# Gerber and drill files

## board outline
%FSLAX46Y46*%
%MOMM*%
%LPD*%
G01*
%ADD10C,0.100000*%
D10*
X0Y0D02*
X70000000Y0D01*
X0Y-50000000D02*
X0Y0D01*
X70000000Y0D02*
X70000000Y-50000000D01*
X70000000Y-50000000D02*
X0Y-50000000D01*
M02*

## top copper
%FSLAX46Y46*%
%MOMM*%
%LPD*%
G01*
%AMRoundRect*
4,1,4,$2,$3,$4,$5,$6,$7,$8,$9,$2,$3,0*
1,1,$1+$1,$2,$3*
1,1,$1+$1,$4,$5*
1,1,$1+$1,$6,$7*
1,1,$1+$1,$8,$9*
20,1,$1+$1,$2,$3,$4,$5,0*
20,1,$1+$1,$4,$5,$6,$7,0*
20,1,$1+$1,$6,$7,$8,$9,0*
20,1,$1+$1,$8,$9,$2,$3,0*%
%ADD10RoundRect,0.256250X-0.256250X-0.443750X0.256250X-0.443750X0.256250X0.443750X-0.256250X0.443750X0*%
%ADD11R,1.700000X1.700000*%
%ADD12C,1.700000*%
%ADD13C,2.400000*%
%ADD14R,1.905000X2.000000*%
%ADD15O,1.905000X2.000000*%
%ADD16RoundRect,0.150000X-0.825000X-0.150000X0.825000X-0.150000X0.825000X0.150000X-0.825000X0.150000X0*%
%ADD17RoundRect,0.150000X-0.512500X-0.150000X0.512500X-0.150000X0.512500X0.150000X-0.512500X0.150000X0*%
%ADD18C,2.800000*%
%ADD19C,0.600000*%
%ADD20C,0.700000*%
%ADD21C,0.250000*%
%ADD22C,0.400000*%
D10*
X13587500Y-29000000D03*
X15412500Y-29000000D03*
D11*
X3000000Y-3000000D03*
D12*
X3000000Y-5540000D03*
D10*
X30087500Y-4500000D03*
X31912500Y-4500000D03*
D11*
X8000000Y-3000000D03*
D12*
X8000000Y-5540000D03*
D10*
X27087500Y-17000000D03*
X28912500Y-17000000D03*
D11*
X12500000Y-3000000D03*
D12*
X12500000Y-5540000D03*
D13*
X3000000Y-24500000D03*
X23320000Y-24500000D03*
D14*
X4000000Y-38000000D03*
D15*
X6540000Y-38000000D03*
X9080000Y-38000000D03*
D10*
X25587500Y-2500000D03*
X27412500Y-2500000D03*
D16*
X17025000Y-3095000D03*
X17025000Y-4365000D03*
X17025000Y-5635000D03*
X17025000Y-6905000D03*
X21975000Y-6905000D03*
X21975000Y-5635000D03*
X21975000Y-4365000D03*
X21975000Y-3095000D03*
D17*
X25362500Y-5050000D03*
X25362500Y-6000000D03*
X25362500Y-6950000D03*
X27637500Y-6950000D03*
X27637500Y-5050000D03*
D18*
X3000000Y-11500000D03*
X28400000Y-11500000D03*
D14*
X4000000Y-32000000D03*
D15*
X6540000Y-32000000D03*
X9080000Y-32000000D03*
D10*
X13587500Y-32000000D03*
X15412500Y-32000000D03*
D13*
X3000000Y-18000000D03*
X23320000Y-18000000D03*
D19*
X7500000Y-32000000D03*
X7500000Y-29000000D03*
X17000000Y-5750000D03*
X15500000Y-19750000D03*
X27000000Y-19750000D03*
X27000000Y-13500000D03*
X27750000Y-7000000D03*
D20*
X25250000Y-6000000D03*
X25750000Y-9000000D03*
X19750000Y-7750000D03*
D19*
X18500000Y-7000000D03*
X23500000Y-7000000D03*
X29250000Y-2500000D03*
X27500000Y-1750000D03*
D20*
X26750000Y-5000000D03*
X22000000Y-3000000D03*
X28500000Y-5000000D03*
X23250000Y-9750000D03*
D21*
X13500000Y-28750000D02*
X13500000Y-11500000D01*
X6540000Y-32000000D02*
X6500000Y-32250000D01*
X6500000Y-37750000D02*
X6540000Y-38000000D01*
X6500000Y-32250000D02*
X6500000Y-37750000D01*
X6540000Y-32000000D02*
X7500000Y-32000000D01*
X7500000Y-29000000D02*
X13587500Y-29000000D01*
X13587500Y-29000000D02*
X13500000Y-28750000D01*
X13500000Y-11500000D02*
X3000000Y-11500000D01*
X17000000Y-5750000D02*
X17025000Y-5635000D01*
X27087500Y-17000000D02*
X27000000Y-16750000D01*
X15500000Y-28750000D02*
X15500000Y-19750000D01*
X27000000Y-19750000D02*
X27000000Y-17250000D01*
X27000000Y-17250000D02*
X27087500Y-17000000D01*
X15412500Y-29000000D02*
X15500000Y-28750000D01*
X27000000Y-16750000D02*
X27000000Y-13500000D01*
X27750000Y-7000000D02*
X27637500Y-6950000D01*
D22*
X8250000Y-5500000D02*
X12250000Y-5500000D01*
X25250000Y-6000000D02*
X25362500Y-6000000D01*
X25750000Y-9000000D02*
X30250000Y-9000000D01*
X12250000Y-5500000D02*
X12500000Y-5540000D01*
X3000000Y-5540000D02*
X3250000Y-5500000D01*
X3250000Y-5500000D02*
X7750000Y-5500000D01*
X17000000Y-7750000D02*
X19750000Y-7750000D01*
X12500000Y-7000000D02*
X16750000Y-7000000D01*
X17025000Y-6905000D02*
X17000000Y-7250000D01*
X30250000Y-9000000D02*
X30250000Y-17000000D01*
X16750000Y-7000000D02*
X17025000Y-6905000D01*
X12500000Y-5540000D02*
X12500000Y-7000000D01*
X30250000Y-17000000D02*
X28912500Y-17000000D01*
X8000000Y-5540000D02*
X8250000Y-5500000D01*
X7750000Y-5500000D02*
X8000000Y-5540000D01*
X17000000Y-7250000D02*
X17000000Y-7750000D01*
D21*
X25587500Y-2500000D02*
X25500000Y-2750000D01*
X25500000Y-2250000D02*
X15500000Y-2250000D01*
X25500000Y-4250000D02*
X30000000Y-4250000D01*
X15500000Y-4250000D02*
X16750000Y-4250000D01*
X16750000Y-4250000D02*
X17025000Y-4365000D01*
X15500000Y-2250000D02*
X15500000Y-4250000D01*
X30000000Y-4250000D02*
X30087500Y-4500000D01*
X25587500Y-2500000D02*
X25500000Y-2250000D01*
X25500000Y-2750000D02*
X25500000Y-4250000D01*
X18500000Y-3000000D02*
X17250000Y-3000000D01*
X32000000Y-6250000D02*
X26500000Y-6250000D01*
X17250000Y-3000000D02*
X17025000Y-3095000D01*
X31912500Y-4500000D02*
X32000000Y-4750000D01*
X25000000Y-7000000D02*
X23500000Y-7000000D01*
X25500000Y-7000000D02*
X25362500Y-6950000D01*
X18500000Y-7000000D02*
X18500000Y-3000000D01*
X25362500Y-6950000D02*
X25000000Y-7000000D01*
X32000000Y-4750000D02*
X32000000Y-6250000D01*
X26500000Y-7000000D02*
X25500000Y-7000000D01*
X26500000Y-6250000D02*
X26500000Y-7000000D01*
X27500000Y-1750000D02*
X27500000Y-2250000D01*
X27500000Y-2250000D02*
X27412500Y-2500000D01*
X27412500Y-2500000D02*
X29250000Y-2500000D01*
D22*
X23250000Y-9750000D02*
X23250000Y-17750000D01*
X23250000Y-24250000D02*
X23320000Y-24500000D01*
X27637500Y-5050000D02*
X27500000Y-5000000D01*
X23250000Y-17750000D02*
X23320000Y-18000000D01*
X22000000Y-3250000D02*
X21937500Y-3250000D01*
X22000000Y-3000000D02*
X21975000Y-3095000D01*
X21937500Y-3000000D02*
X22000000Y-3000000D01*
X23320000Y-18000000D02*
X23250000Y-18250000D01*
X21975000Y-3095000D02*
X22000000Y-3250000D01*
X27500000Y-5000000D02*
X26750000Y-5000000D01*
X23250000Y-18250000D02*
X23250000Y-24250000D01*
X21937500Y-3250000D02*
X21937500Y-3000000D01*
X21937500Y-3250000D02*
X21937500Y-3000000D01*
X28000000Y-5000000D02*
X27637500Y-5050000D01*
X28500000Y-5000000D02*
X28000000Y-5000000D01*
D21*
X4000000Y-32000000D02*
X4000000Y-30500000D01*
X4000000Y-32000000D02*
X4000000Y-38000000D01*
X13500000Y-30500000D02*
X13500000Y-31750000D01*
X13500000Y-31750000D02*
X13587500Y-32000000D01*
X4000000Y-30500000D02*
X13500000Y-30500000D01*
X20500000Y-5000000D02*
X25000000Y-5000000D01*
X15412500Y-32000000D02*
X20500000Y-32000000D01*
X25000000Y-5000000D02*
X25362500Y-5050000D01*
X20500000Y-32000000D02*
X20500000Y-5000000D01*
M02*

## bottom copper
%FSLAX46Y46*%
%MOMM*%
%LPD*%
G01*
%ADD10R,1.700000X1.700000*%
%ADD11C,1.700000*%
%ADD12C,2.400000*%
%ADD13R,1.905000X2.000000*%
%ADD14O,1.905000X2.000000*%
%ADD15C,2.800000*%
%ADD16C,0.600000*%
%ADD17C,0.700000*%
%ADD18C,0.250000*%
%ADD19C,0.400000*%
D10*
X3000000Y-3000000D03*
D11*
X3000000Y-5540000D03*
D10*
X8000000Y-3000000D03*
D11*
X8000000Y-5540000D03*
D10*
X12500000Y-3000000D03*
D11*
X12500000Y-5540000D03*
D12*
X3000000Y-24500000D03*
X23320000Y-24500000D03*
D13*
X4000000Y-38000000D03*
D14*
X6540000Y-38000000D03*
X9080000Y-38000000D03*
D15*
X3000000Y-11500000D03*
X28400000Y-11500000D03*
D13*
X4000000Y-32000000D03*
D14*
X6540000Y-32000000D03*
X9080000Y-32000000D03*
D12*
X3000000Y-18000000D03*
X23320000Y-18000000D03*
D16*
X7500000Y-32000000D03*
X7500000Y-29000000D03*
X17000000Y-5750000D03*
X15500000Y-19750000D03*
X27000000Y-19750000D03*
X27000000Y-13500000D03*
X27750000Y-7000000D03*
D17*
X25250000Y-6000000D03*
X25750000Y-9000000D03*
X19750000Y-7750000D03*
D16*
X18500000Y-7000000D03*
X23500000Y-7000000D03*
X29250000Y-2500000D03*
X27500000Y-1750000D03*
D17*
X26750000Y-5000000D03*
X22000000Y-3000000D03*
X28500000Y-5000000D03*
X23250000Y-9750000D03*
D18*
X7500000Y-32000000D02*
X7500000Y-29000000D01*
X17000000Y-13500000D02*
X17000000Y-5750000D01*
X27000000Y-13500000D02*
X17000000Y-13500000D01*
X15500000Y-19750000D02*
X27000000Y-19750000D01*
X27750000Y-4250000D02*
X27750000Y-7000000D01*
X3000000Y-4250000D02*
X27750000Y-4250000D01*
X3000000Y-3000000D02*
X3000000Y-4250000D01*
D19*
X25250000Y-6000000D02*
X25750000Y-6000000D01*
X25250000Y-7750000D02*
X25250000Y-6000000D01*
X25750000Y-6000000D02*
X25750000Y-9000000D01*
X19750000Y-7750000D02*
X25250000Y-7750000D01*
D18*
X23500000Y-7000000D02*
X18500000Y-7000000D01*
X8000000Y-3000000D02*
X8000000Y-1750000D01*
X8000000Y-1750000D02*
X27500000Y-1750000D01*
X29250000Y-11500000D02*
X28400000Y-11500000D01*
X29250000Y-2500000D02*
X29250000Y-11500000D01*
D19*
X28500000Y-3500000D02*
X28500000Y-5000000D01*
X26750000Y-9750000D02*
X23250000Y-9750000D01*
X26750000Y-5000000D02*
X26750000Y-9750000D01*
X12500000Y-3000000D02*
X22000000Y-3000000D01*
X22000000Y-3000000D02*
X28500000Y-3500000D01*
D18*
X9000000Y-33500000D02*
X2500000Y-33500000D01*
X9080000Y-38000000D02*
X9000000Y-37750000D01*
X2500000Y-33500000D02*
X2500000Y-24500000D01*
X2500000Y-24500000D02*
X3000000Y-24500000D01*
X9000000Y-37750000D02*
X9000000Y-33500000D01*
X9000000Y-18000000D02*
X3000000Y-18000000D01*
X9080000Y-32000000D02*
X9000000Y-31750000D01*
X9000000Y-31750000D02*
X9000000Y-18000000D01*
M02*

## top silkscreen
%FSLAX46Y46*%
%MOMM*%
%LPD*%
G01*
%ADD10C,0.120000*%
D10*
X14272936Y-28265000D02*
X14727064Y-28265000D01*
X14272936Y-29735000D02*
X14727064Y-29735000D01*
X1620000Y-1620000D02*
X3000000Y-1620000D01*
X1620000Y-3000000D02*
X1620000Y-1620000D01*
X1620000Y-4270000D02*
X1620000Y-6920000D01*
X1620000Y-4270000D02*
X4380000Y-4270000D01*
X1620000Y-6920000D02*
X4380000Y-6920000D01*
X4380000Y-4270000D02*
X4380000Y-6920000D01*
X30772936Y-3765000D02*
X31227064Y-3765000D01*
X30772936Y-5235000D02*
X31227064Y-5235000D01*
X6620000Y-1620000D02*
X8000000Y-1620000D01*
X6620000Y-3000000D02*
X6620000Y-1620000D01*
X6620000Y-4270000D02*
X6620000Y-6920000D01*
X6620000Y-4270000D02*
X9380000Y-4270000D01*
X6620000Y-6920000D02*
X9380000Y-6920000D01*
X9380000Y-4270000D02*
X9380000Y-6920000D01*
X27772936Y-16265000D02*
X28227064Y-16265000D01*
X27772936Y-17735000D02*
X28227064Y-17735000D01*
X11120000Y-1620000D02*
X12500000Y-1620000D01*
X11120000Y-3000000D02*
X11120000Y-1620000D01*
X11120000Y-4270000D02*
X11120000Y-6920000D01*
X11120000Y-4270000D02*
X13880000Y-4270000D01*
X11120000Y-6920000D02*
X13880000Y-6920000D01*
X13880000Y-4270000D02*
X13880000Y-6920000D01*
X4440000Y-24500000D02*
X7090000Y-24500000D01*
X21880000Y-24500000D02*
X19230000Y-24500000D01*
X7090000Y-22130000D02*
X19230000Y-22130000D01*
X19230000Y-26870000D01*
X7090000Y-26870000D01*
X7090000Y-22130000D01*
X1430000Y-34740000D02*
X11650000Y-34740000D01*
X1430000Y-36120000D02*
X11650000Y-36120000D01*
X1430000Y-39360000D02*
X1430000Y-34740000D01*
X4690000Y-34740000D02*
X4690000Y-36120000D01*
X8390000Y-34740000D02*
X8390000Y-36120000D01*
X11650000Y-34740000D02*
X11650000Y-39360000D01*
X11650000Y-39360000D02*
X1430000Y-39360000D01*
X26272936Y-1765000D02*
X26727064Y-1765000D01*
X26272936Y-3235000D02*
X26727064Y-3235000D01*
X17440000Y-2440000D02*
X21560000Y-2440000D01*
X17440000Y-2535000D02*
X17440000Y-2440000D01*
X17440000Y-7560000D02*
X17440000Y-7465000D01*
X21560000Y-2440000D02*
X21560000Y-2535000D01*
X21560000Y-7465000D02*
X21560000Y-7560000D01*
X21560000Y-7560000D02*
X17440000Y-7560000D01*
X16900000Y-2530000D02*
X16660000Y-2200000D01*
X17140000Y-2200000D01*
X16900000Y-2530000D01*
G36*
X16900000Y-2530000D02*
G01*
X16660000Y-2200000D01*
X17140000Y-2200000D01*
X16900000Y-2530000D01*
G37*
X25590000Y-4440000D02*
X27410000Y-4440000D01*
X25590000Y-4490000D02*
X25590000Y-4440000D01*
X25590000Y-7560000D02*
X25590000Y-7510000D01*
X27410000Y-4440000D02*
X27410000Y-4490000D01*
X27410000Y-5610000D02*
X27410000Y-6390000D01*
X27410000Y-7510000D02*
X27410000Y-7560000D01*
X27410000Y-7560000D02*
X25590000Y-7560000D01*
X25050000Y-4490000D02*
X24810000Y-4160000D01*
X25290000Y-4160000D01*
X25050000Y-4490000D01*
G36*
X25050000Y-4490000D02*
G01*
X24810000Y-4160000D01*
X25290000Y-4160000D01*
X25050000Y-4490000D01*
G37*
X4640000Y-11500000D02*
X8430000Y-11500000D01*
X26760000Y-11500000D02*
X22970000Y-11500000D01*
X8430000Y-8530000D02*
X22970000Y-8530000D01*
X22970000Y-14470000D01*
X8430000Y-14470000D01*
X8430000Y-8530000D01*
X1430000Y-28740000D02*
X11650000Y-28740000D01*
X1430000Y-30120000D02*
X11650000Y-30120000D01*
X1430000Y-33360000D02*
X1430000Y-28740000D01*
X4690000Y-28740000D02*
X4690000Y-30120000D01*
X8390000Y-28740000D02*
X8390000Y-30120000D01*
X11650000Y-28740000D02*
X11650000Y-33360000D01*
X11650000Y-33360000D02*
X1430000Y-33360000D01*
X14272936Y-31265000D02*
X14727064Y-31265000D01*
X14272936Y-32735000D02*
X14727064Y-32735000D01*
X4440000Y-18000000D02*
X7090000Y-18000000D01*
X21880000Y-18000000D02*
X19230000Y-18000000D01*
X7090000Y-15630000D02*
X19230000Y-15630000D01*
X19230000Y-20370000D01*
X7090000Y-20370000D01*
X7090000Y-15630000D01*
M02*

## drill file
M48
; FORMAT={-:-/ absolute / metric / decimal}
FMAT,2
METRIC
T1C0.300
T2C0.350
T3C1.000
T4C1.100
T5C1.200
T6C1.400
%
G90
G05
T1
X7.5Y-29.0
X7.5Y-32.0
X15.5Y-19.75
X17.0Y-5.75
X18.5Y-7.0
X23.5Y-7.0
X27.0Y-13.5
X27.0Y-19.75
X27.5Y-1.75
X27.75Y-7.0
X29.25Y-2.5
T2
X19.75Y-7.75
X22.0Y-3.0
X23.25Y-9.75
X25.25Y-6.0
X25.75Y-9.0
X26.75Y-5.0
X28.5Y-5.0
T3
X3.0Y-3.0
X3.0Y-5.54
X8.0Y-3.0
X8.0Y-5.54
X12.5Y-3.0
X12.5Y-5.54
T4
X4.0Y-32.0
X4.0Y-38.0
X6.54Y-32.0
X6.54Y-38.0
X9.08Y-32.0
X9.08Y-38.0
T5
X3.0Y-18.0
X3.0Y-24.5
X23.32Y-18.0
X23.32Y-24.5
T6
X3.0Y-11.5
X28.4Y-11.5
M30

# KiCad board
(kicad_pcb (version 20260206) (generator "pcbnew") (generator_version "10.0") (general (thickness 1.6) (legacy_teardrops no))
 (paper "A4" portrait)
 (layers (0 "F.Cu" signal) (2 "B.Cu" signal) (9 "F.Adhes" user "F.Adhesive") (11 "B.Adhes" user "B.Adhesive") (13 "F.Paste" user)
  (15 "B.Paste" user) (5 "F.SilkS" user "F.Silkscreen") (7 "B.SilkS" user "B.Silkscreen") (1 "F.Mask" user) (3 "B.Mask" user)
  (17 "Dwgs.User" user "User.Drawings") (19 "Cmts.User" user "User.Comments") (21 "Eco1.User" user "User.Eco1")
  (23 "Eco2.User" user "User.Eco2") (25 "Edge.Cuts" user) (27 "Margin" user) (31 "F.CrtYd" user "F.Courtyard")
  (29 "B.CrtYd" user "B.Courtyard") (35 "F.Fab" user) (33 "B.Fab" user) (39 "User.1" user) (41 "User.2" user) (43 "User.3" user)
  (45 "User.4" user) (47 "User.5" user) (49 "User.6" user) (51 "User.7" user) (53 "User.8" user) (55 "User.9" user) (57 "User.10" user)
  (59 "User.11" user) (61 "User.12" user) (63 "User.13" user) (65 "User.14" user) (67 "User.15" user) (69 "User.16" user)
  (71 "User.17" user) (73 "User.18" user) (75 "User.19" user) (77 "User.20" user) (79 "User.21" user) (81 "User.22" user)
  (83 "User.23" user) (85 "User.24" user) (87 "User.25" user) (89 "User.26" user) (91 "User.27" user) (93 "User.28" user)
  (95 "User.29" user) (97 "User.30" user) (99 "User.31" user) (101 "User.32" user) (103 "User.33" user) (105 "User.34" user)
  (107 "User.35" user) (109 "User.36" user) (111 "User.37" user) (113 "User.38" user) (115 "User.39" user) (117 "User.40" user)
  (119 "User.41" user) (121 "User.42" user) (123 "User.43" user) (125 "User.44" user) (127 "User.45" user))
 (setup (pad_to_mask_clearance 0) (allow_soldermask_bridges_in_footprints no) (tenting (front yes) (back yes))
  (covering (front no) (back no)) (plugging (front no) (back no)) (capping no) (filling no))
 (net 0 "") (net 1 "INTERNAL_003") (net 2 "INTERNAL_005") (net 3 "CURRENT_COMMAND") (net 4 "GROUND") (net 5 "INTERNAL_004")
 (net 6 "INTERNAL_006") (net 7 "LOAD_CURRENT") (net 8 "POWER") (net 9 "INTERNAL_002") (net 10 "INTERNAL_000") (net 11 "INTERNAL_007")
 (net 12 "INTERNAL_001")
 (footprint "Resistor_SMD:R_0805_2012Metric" (layer "F.Cu") (at 14.5 29)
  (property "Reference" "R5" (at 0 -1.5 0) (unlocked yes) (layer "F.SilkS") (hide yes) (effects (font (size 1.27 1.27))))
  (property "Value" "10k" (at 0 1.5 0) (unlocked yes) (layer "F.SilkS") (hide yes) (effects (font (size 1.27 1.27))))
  (fp_line (start -0.227064 -0.735) (end 0.227064 -0.735) (stroke (width 0.12) (type solid)) (layer "F.SilkS"))
  (fp_line (start -0.227064 0.735) (end 0.227064 0.735) (stroke (width 0.12) (type solid)) (layer "F.SilkS"))
  (pad "1" smd roundrect (at -0.9125 0) (size 1.025 1.4) (layers "F.Cu" "F.Mask" "F.Paste") (roundrect_rratio 0.25) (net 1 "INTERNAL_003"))
  (pad "2" smd roundrect (at 0.9125 0) (size 1.025 1.4) (layers "F.Cu" "F.Mask" "F.Paste") (roundrect_rratio 0.25) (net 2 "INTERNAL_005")))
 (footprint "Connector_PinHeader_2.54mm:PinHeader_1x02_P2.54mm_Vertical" (layer "F.Cu") (at 3 3)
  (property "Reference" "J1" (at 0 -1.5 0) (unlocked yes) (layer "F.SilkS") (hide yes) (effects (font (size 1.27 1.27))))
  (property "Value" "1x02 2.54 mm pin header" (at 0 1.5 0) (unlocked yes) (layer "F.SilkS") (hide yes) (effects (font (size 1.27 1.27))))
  (fp_line (start -1.38 -1.38) (end 0 -1.38) (stroke (width 0.12) (type solid)) (layer "F.SilkS"))
  (fp_line (start -1.38 0) (end -1.38 -1.38) (stroke (width 0.12) (type solid)) (layer "F.SilkS"))
  (fp_line (start -1.38 1.27) (end -1.38 3.92) (stroke (width 0.12) (type solid)) (layer "F.SilkS"))
  (fp_line (start -1.38 1.27) (end 1.38 1.27) (stroke (width 0.12) (type solid)) (layer "F.SilkS"))
  (fp_line (start -1.38 3.92) (end 1.38 3.92) (stroke (width 0.12) (type solid)) (layer "F.SilkS"))
  (fp_line (start 1.38 1.27) (end 1.38 3.92) (stroke (width 0.12) (type solid)) (layer "F.SilkS"))
  (pad "1" thru_hole rect (at 0 0) (size 1.7 1.7) (drill 1) (layers "*.Cu" "*.Mask") (remove_unused_layers no) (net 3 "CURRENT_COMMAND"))
  (pad "2" thru_hole circle (at 0 2.54) (size 1.7 1.7) (drill 1) (layers "*.Cu" "*.Mask") (remove_unused_layers no) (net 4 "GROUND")))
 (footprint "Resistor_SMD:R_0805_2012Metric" (layer "F.Cu") (at 31 4.5)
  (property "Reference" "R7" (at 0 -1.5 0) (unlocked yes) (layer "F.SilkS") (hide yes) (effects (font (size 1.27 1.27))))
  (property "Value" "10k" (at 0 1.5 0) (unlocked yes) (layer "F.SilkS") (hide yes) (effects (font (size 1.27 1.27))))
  (fp_line (start -0.227064 -0.735) (end 0.227064 -0.735) (stroke (width 0.12) (type solid)) (layer "F.SilkS"))
  (fp_line (start -0.227064 0.735) (end 0.227064 0.735) (stroke (width 0.12) (type solid)) (layer "F.SilkS"))
  (pad "1" smd roundrect (at -0.9125 0) (size 1.025 1.4) (layers "F.Cu" "F.Mask" "F.Paste") (roundrect_rratio 0.25) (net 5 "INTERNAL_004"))
  (pad "2" smd roundrect (at 0.9125 0) (size 1.025 1.4) (layers "F.Cu" "F.Mask" "F.Paste") (roundrect_rratio 0.25) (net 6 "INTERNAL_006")))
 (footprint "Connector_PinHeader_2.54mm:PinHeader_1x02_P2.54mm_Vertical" (layer "F.Cu") (at 8 3)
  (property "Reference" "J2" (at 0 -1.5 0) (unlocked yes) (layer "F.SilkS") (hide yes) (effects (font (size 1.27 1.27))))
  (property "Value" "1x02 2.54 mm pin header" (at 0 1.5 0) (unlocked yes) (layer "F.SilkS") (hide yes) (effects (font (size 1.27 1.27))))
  (fp_line (start -1.38 -1.38) (end 0 -1.38) (stroke (width 0.12) (type solid)) (layer "F.SilkS"))
  (fp_line (start -1.38 0) (end -1.38 -1.38) (stroke (width 0.12) (type solid)) (layer "F.SilkS"))
  (fp_line (start -1.38 1.27) (end -1.38 3.92) (stroke (width 0.12) (type solid)) (layer "F.SilkS"))
  (fp_line (start -1.38 1.27) (end 1.38 1.27) (stroke (width 0.12) (type solid)) (layer "F.SilkS"))
  (fp_line (start -1.38 3.92) (end 1.38 3.92) (stroke (width 0.12) (type solid)) (layer "F.SilkS"))
  (fp_line (start 1.38 1.27) (end 1.38 3.92) (stroke (width 0.12) (type solid)) (layer "F.SilkS"))
  (pad "1" thru_hole rect (at 0 0) (size 1.7 1.7) (drill 1) (layers "*.Cu" "*.Mask") (remove_unused_layers no) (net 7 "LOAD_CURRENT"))
  (pad "2" thru_hole circle (at 0 2.54) (size 1.7 1.7) (drill 1) (layers "*.Cu" "*.Mask") (remove_unused_layers no) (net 4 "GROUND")))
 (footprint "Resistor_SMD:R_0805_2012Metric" (layer "F.Cu") (at 28 17)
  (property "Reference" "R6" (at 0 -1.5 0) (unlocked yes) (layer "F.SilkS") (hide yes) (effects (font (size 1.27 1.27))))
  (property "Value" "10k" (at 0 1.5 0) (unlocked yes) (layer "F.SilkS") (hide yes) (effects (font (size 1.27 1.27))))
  (fp_line (start -0.227064 -0.735) (end 0.227064 -0.735) (stroke (width 0.12) (type solid)) (layer "F.SilkS"))
  (fp_line (start -0.227064 0.735) (end 0.227064 0.735) (stroke (width 0.12) (type solid)) (layer "F.SilkS"))
  (pad "1" smd roundrect (at -0.9125 0) (size 1.025 1.4) (layers "F.Cu" "F.Mask" "F.Paste") (roundrect_rratio 0.25) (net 2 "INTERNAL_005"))
  (pad "2" smd roundrect (at 0.9125 0) (size 1.025 1.4) (layers "F.Cu" "F.Mask" "F.Paste") (roundrect_rratio 0.25) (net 4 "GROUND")))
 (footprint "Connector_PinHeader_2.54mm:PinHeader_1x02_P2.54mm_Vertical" (layer "F.Cu") (at 12.5 3)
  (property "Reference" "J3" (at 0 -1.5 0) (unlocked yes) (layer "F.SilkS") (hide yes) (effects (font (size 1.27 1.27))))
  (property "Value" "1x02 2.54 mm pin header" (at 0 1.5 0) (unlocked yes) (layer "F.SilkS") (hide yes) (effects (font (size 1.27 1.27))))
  (fp_line (start -1.38 -1.38) (end 0 -1.38) (stroke (width 0.12) (type solid)) (layer "F.SilkS"))
  (fp_line (start -1.38 0) (end -1.38 -1.38) (stroke (width 0.12) (type solid)) (layer "F.SilkS"))
  (fp_line (start -1.38 1.27) (end -1.38 3.92) (stroke (width 0.12) (type solid)) (layer "F.SilkS"))
  (fp_line (start -1.38 1.27) (end 1.38 1.27) (stroke (width 0.12) (type solid)) (layer "F.SilkS"))
  (fp_line (start -1.38 3.92) (end 1.38 3.92) (stroke (width 0.12) (type solid)) (layer "F.SilkS"))
  (fp_line (start 1.38 1.27) (end 1.38 3.92) (stroke (width 0.12) (type solid)) (layer "F.SilkS"))
  (pad "1" thru_hole rect (at 0 0) (size 1.7 1.7) (drill 1) (layers "*.Cu" "*.Mask") (remove_unused_layers no) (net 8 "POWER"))
  (pad "2" thru_hole circle (at 0 2.54) (size 1.7 1.7) (drill 1) (layers "*.Cu" "*.Mask") (remove_unused_layers no) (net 4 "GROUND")))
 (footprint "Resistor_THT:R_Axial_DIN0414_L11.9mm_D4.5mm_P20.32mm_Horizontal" (layer "F.Cu") (at 3 24.5)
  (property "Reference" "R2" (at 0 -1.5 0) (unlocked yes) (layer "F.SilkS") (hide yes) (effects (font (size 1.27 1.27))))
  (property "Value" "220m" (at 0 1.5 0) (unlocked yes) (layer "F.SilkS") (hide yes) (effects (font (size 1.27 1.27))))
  (fp_line (start 1.44 0) (end 4.09 0) (stroke (width 0.12) (type solid)) (layer "F.SilkS"))
  (fp_line (start 18.88 0) (end 16.23 0) (stroke (width 0.12) (type solid)) (layer "F.SilkS"))
  (fp_rect (start 4.09 -2.37) (end 16.23 2.37) (stroke (width 0.12) (type solid)) (fill no) (layer "F.SilkS"))
  (pad "1" thru_hole circle (at 0 0) (size 2.4 2.4) (drill 1.2) (layers "*.Cu" "*.Mask") (remove_unused_layers no) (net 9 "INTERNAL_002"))
  (pad "2" thru_hole circle (at 20.32 0) (size 2.4 2.4) (drill 1.2) (layers "*.Cu" "*.Mask") (remove_unused_layers no) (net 8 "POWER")))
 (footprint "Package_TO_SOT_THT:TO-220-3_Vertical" (layer "F.Cu") (at 4 38)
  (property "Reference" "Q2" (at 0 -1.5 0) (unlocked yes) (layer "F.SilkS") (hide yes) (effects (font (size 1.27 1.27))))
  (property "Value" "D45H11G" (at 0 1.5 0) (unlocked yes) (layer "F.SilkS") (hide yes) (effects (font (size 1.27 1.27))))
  (fp_line (start -2.57 -3.26) (end 7.65 -3.26) (stroke (width 0.12) (type solid)) (layer "F.SilkS"))
  (fp_line (start -2.57 -1.88) (end 7.65 -1.88) (stroke (width 0.12) (type solid)) (layer "F.SilkS"))
  (fp_line (start -2.57 1.36) (end -2.57 -3.26) (stroke (width 0.12) (type solid)) (layer "F.SilkS"))
  (fp_line (start 0.69 -3.26) (end 0.69 -1.88) (stroke (width 0.12) (type solid)) (layer "F.SilkS"))
  (fp_line (start 4.39 -3.26) (end 4.39 -1.88) (stroke (width 0.12) (type solid)) (layer "F.SilkS"))
  (fp_line (start 7.65 -3.26) (end 7.65 1.36) (stroke (width 0.12) (type solid)) (layer "F.SilkS"))
  (fp_line (start 7.65 1.36) (end -2.57 1.36) (stroke (width 0.12) (type solid)) (layer "F.SilkS"))
  (pad "1" thru_hole rect (at 0 0) (size 1.905 2) (drill 1.1) (layers "*.Cu" "*.Mask") (remove_unused_layers no) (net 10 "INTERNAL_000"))
  (pad "2" thru_hole oval (at 2.54 0) (size 1.905 2) (drill 1.1) (layers "*.Cu" "*.Mask") (remove_unused_layers no) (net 1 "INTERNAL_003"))
  (pad "3" thru_hole oval (at 5.08 0) (size 1.905 2) (drill 1.1) (layers "*.Cu" "*.Mask") (remove_unused_layers no) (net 9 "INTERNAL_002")))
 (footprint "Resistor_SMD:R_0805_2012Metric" (layer "F.Cu") (at 26.5 2.5)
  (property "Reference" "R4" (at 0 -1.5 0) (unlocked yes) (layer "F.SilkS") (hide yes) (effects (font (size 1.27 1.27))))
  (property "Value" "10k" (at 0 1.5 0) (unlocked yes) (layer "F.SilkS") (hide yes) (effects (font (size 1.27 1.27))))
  (fp_line (start -0.227064 -0.735) (end 0.227064 -0.735) (stroke (width 0.12) (type solid)) (layer "F.SilkS"))
  (fp_line (start -0.227064 0.735) (end 0.227064 0.735) (stroke (width 0.12) (type solid)) (layer "F.SilkS"))
  (pad "1" smd roundrect (at -0.9125 0) (size 1.025 1.4) (layers "F.Cu" "F.Mask" "F.Paste") (roundrect_rratio 0.25) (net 5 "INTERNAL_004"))
  (pad "2" smd roundrect (at 0.9125 0) (size 1.025 1.4) (layers "F.Cu" "F.Mask" "F.Paste") (roundrect_rratio 0.25) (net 7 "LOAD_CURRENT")))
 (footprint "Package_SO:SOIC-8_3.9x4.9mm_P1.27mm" (layer "F.Cu") (at 19.5 5)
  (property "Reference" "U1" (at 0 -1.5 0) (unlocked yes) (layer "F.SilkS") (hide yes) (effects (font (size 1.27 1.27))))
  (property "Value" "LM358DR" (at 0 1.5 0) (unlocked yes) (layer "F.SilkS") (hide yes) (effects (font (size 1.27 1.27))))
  (fp_line (start -2.06 -2.56) (end 2.06 -2.56) (stroke (width 0.12) (type solid)) (layer "F.SilkS"))
  (fp_line (start -2.06 -2.465) (end -2.06 -2.56) (stroke (width 0.12) (type solid)) (layer "F.SilkS"))
  (fp_line (start -2.06 2.56) (end -2.06 2.465) (stroke (width 0.12) (type solid)) (layer "F.SilkS"))
  (fp_line (start 2.06 -2.56) (end 2.06 -2.465) (stroke (width 0.12) (type solid)) (layer "F.SilkS"))
  (fp_line (start 2.06 2.465) (end 2.06 2.56) (stroke (width 0.12) (type solid)) (layer "F.SilkS"))
  (fp_line (start 2.06 2.56) (end -2.06 2.56) (stroke (width 0.12) (type solid)) (layer "F.SilkS"))
  (fp_poly (pts (xy -2.6 -2.47) (xy -2.84 -2.8) (xy -2.36 -2.8)) (stroke (width 0.12) (type solid)) (fill yes) (layer "F.SilkS"))
  (pad "1" smd roundrect (at -2.475 -1.905) (size 1.95 0.6) (layers "F.Cu" "F.Mask" "F.Paste") (roundrect_rratio 0.25)
   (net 6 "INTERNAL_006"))
  (pad "2" smd roundrect (at -2.475 -0.635) (size 1.95 0.6) (layers "F.Cu" "F.Mask" "F.Paste") (roundrect_rratio 0.25)
   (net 5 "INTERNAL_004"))
  (pad "3" smd roundrect (at -2.475 0.635) (size 1.95 0.6) (layers "F.Cu" "F.Mask" "F.Paste") (roundrect_rratio 0.25) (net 2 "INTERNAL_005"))
  (pad "4" smd roundrect (at -2.475 1.905) (size 1.95 0.6) (layers "F.Cu" "F.Mask" "F.Paste") (roundrect_rratio 0.25) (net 4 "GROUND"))
  (pad "5" smd roundrect (at 2.475 1.905) (size 1.95 0.6) (layers "F.Cu" "F.Mask" "F.Paste") (roundrect_rratio 0.25))
  (pad "6" smd roundrect (at 2.475 0.635) (size 1.95 0.6) (layers "F.Cu" "F.Mask" "F.Paste") (roundrect_rratio 0.25))
  (pad "7" smd roundrect (at 2.475 -0.635) (size 1.95 0.6) (layers "F.Cu" "F.Mask" "F.Paste") (roundrect_rratio 0.25))
  (pad "8" smd roundrect (at 2.475 -1.905) (size 1.95 0.6) (layers "F.Cu" "F.Mask" "F.Paste") (roundrect_rratio 0.25) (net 8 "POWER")))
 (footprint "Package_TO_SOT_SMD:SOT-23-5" (layer "F.Cu") (at 26.5 6)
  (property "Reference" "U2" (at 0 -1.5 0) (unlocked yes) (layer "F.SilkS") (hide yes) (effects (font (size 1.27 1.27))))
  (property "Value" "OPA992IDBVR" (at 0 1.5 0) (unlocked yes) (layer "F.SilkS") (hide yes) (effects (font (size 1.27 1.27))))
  (fp_line (start -0.91 -1.56) (end 0.91 -1.56) (stroke (width 0.12) (type solid)) (layer "F.SilkS"))
  (fp_line (start -0.91 -1.51) (end -0.91 -1.56) (stroke (width 0.12) (type solid)) (layer "F.SilkS"))
  (fp_line (start -0.91 1.56) (end -0.91 1.51) (stroke (width 0.12) (type solid)) (layer "F.SilkS"))
  (fp_line (start 0.91 -1.56) (end 0.91 -1.51) (stroke (width 0.12) (type solid)) (layer "F.SilkS"))
  (fp_line (start 0.91 -0.39) (end 0.91 0.39) (stroke (width 0.12) (type solid)) (layer "F.SilkS"))
  (fp_line (start 0.91 1.51) (end 0.91 1.56) (stroke (width 0.12) (type solid)) (layer "F.SilkS"))
  (fp_line (start 0.91 1.56) (end -0.91 1.56) (stroke (width 0.12) (type solid)) (layer "F.SilkS"))
  (fp_poly (pts (xy -1.45 -1.51) (xy -1.69 -1.84) (xy -1.21 -1.84)) (stroke (width 0.12) (type solid)) (fill yes) (layer "F.SilkS"))
  (pad "1" smd roundrect (at -1.1375 -0.95) (size 1.325 0.6) (layers "F.Cu" "F.Mask" "F.Paste") (roundrect_rratio 0.25)
   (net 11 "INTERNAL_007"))
  (pad "2" smd roundrect (at -1.1375 0) (size 1.325 0.6) (layers "F.Cu" "F.Mask" "F.Paste") (roundrect_rratio 0.25) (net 4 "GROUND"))
  (pad "3" smd roundrect (at -1.1375 0.95) (size 1.325 0.6) (layers "F.Cu" "F.Mask" "F.Paste") (roundrect_rratio 0.25)
   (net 6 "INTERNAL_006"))
  (pad "4" smd roundrect (at 1.1375 0.95) (size 1.325 0.6) (layers "F.Cu" "F.Mask" "F.Paste") (roundrect_rratio 0.25)
   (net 3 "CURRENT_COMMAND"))
  (pad "5" smd roundrect (at 1.1375 -0.95) (size 1.325 0.6) (layers "F.Cu" "F.Mask" "F.Paste") (roundrect_rratio 0.25) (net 8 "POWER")))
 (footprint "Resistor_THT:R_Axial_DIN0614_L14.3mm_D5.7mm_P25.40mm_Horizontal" (layer "F.Cu") (at 3 11.5)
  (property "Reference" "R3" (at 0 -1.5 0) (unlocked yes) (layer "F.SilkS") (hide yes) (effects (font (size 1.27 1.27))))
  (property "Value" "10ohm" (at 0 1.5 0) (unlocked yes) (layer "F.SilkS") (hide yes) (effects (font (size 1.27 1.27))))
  (fp_line (start 1.64 0) (end 5.43 0) (stroke (width 0.12) (type solid)) (layer "F.SilkS"))
  (fp_line (start 23.76 0) (end 19.97 0) (stroke (width 0.12) (type solid)) (layer "F.SilkS"))
  (fp_rect (start 5.43 -2.97) (end 19.97 2.97) (stroke (width 0.12) (type solid)) (fill no) (layer "F.SilkS"))
  (pad "1" thru_hole circle (at 0 0) (size 2.8 2.8) (drill 1.4) (layers "*.Cu" "*.Mask") (remove_unused_layers no) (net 1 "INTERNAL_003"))
  (pad "2" thru_hole circle (at 25.4 0) (size 2.8 2.8) (drill 1.4) (layers "*.Cu" "*.Mask") (remove_unused_layers no) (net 7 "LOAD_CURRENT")))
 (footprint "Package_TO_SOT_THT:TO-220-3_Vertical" (layer "F.Cu") (at 4 32)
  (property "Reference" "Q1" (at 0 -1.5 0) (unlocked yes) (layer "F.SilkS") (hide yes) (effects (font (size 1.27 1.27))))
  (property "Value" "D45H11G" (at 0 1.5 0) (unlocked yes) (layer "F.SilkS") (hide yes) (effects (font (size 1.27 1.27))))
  (fp_line (start -2.57 -3.26) (end 7.65 -3.26) (stroke (width 0.12) (type solid)) (layer "F.SilkS"))
  (fp_line (start -2.57 -1.88) (end 7.65 -1.88) (stroke (width 0.12) (type solid)) (layer "F.SilkS"))
  (fp_line (start -2.57 1.36) (end -2.57 -3.26) (stroke (width 0.12) (type solid)) (layer "F.SilkS"))
  (fp_line (start 0.69 -3.26) (end 0.69 -1.88) (stroke (width 0.12) (type solid)) (layer "F.SilkS"))
  (fp_line (start 4.39 -3.26) (end 4.39 -1.88) (stroke (width 0.12) (type solid)) (layer "F.SilkS"))
  (fp_line (start 7.65 -3.26) (end 7.65 1.36) (stroke (width 0.12) (type solid)) (layer "F.SilkS"))
  (fp_line (start 7.65 1.36) (end -2.57 1.36) (stroke (width 0.12) (type solid)) (layer "F.SilkS"))
  (pad "1" thru_hole rect (at 0 0) (size 1.905 2) (drill 1.1) (layers "*.Cu" "*.Mask") (remove_unused_layers no) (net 10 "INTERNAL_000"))
  (pad "2" thru_hole oval (at 2.54 0) (size 1.905 2) (drill 1.1) (layers "*.Cu" "*.Mask") (remove_unused_layers no) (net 1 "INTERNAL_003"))
  (pad "3" thru_hole oval (at 5.08 0) (size 1.905 2) (drill 1.1) (layers "*.Cu" "*.Mask") (remove_unused_layers no) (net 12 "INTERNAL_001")))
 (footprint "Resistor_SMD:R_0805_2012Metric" (layer "F.Cu") (at 14.5 32)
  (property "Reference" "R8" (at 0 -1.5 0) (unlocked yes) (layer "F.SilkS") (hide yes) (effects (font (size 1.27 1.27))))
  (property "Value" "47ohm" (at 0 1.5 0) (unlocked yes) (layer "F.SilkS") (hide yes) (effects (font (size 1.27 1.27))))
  (fp_line (start -0.227064 -0.735) (end 0.227064 -0.735) (stroke (width 0.12) (type solid)) (layer "F.SilkS"))
  (fp_line (start -0.227064 0.735) (end 0.227064 0.735) (stroke (width 0.12) (type solid)) (layer "F.SilkS"))
  (pad "1" smd roundrect (at -0.9125 0) (size 1.025 1.4) (layers "F.Cu" "F.Mask" "F.Paste") (roundrect_rratio 0.25) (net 10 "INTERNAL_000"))
  (pad "2" smd roundrect (at 0.9125 0) (size 1.025 1.4) (layers "F.Cu" "F.Mask" "F.Paste") (roundrect_rratio 0.25) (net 11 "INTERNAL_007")))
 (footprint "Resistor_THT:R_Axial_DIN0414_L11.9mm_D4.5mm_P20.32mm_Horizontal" (layer "F.Cu") (at 3 18)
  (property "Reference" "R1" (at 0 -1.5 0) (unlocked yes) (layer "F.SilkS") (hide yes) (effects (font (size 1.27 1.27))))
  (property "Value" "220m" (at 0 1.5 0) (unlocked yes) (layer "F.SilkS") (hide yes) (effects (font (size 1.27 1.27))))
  (fp_line (start 1.44 0) (end 4.09 0) (stroke (width 0.12) (type solid)) (layer "F.SilkS"))
  (fp_line (start 18.88 0) (end 16.23 0) (stroke (width 0.12) (type solid)) (layer "F.SilkS"))
  (fp_rect (start 4.09 -2.37) (end 16.23 2.37) (stroke (width 0.12) (type solid)) (fill no) (layer "F.SilkS"))
  (pad "1" thru_hole circle (at 0 0) (size 2.4 2.4) (drill 1.2) (layers "*.Cu" "*.Mask") (remove_unused_layers no) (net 12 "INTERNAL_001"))
  (pad "2" thru_hole circle (at 20.32 0) (size 2.4 2.4) (drill 1.2) (layers "*.Cu" "*.Mask") (remove_unused_layers no) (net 8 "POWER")))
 (gr_line (start 0 0) (end 70 0) (stroke (width 0.1) (type solid)) (layer "Edge.Cuts"))
 (gr_line (start 0 50) (end 0 0) (stroke (width 0.1) (type solid)) (layer "Edge.Cuts"))
 (gr_line (start 70 0) (end 70 50) (stroke (width 0.1) (type solid)) (layer "Edge.Cuts"))
 (gr_line (start 70 50) (end 0 50) (stroke (width 0.1) (type solid)) (layer "Edge.Cuts"))
 (segment (start 13.5 28.75) (end 13.5 11.5) (width 0.25) (layer "F.Cu") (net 1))
 (segment (start 6.54 32) (end 6.5 32.25) (width 0.25) (layer "F.Cu") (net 1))
 (segment (start 6.5 37.75) (end 6.54 38) (width 0.25) (layer "F.Cu") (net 1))
 (segment (start 6.5 32.25) (end 6.5 37.75) (width 0.25) (layer "F.Cu") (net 1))
 (segment (start 6.54 32) (end 7.5 32) (width 0.25) (layer "F.Cu") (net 1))
 (segment (start 7.5 29) (end 13.5875 29) (width 0.25) (layer "F.Cu") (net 1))
 (segment (start 13.5875 29) (end 13.5 28.75) (width 0.25) (layer "F.Cu") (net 1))
 (segment (start 13.5 11.5) (end 3 11.5) (width 0.25) (layer "F.Cu") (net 1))
 (via (at 7.5 32) (size 0.6) (drill 0.3) (layers "F.Cu" "B.Cu") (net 1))
 (via (at 7.5 29) (size 0.6) (drill 0.3) (layers "F.Cu" "B.Cu") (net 1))
 (segment (start 7.5 32) (end 7.5 29) (width 0.25) (layer "B.Cu") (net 1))
 (segment (start 17 5.75) (end 17.025 5.635) (width 0.25) (layer "F.Cu") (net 2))
 (segment (start 27.0875 17) (end 27 16.75) (width 0.25) (layer "F.Cu") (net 2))
 (segment (start 15.5 28.75) (end 15.5 19.75) (width 0.25) (layer "F.Cu") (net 2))
 (segment (start 27 19.75) (end 27 17.25) (width 0.25) (layer "F.Cu") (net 2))
 (segment (start 27 17.25) (end 27.0875 17) (width 0.25) (layer "F.Cu") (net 2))
 (segment (start 15.4125 29) (end 15.5 28.75) (width 0.25) (layer "F.Cu") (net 2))
 (segment (start 27 16.75) (end 27 13.5) (width 0.25) (layer "F.Cu") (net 2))
 (via (at 17 5.75) (size 0.6) (drill 0.3) (layers "F.Cu" "B.Cu") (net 2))
 (via (at 15.5 19.75) (size 0.6) (drill 0.3) (layers "F.Cu" "B.Cu") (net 2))
 (via (at 27 19.75) (size 0.6) (drill 0.3) (layers "F.Cu" "B.Cu") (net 2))
 (via (at 27 13.5) (size 0.6) (drill 0.3) (layers "F.Cu" "B.Cu") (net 2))
 (segment (start 17 13.5) (end 17 5.75) (width 0.25) (layer "B.Cu") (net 2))
 (segment (start 27 13.5) (end 17 13.5) (width 0.25) (layer "B.Cu") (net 2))
 (segment (start 15.5 19.75) (end 27 19.75) (width 0.25) (layer "B.Cu") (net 2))
 (segment (start 27.75 7) (end 27.6375 6.95) (width 0.25) (layer "F.Cu") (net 3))
 (via (at 27.75 7) (size 0.6) (drill 0.3) (layers "F.Cu" "B.Cu") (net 3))
 (segment (start 27.75 4.25) (end 27.75 7) (width 0.25) (layer "B.Cu") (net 3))
 (segment (start 3 4.25) (end 27.75 4.25) (width 0.25) (layer "B.Cu") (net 3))
 (segment (start 3 3) (end 3 4.25) (width 0.25) (layer "B.Cu") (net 3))
 (segment (start 8.25 5.5) (end 12.25 5.5) (width 0.4) (layer "F.Cu") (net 4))
 (segment (start 25.25 6) (end 25.3625 6) (width 0.4) (layer "F.Cu") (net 4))
 (segment (start 25.75 9) (end 30.25 9) (width 0.4) (layer "F.Cu") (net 4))
 (segment (start 12.25 5.5) (end 12.5 5.54) (width 0.4) (layer "F.Cu") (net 4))
 (segment (start 3 5.54) (end 3.25 5.5) (width 0.4) (layer "F.Cu") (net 4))
 (segment (start 3.25 5.5) (end 7.75 5.5) (width 0.4) (layer "F.Cu") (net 4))
 (segment (start 17 7.75) (end 19.75 7.75) (width 0.4) (layer "F.Cu") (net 4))
 (segment (start 12.5 7) (end 16.75 7) (width 0.4) (layer "F.Cu") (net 4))
 (segment (start 17.025 6.905) (end 17 7.25) (width 0.4) (layer "F.Cu") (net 4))
 (segment (start 30.25 9) (end 30.25 17) (width 0.4) (layer "F.Cu") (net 4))
 (segment (start 16.75 7) (end 17.025 6.905) (width 0.4) (layer "F.Cu") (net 4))
 (segment (start 12.5 5.54) (end 12.5 7) (width 0.4) (layer "F.Cu") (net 4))
 (segment (start 30.25 17) (end 28.9125 17) (width 0.4) (layer "F.Cu") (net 4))
 (segment (start 8 5.54) (end 8.25 5.5) (width 0.4) (layer "F.Cu") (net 4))
 (segment (start 7.75 5.5) (end 8 5.54) (width 0.4) (layer "F.Cu") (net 4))
 (segment (start 17 7.25) (end 17 7.75) (width 0.4) (layer "F.Cu") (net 4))
 (via (at 25.25 6) (size 0.7) (drill 0.35) (layers "F.Cu" "B.Cu") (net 4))
 (via (at 25.75 9) (size 0.7) (drill 0.35) (layers "F.Cu" "B.Cu") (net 4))
 (via (at 19.75 7.75) (size 0.7) (drill 0.35) (layers "F.Cu" "B.Cu") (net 4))
 (segment (start 25.25 6) (end 25.75 6) (width 0.4) (layer "B.Cu") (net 4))
 (segment (start 25.25 7.75) (end 25.25 6) (width 0.4) (layer "B.Cu") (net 4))
 (segment (start 25.75 6) (end 25.75 9) (width 0.4) (layer "B.Cu") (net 4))
 (segment (start 19.75 7.75) (end 25.25 7.75) (width 0.4) (layer "B.Cu") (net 4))
 (segment (start 25.5875 2.5) (end 25.5 2.75) (width 0.25) (layer "F.Cu") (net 5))
 (segment (start 25.5 2.25) (end 15.5 2.25) (width 0.25) (layer "F.Cu") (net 5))
 (segment (start 25.5 4.25) (end 30 4.25) (width 0.25) (layer "F.Cu") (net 5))
 (segment (start 15.5 4.25) (end 16.75 4.25) (width 0.25) (layer "F.Cu") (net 5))
 (segment (start 16.75 4.25) (end 17.025 4.365) (width 0.25) (layer "F.Cu") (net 5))
 (segment (start 15.5 2.25) (end 15.5 4.25) (width 0.25) (layer "F.Cu") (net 5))
 (segment (start 30 4.25) (end 30.0875 4.5) (width 0.25) (layer "F.Cu") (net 5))
 (segment (start 25.5875 2.5) (end 25.5 2.25) (width 0.25) (layer "F.Cu") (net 5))
 (segment (start 25.5 2.75) (end 25.5 4.25) (width 0.25) (layer "F.Cu") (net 5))
 (segment (start 18.5 3) (end 17.25 3) (width 0.25) (layer "F.Cu") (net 6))
 (segment (start 32 6.25) (end 26.5 6.25) (width 0.25) (layer "F.Cu") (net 6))
 (segment (start 17.25 3) (end 17.025 3.095) (width 0.25) (layer "F.Cu") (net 6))
 (segment (start 31.9125 4.5) (end 32 4.75) (width 0.25) (layer "F.Cu") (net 6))
 (segment (start 25 7) (end 23.5 7) (width 0.25) (layer "F.Cu") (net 6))
 (segment (start 25.5 7) (end 25.3625 6.95) (width 0.25) (layer "F.Cu") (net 6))
 (segment (start 18.5 7) (end 18.5 3) (width 0.25) (layer "F.Cu") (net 6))
 (segment (start 25.3625 6.95) (end 25 7) (width 0.25) (layer "F.Cu") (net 6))
 (segment (start 32 4.75) (end 32 6.25) (width 0.25) (layer "F.Cu") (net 6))
 (segment (start 26.5 7) (end 25.5 7) (width 0.25) (layer "F.Cu") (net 6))
 (segment (start 26.5 6.25) (end 26.5 7) (width 0.25) (layer "F.Cu") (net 6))
 (via (at 18.5 7) (size 0.6) (drill 0.3) (layers "F.Cu" "B.Cu") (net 6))
 (via (at 23.5 7) (size 0.6) (drill 0.3) (layers "F.Cu" "B.Cu") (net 6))
 (segment (start 23.5 7) (end 18.5 7) (width 0.25) (layer "B.Cu") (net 6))
 (segment (start 27.5 1.75) (end 27.5 2.25) (width 0.25) (layer "F.Cu") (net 7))
 (segment (start 27.5 2.25) (end 27.4125 2.5) (width 0.25) (layer "F.Cu") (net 7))
 (segment (start 27.4125 2.5) (end 29.25 2.5) (width 0.25) (layer "F.Cu") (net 7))
 (via (at 29.25 2.5) (size 0.6) (drill 0.3) (layers "F.Cu" "B.Cu") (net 7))
 (via (at 27.5 1.75) (size 0.6) (drill 0.3) (layers "F.Cu" "B.Cu") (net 7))
 (segment (start 8 3) (end 8 1.75) (width 0.25) (layer "B.Cu") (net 7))
 (segment (start 8 1.75) (end 27.5 1.75) (width 0.25) (layer "B.Cu") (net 7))
 (segment (start 29.25 11.5) (end 28.4 11.5) (width 0.25) (layer "B.Cu") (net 7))
 (segment (start 29.25 2.5) (end 29.25 11.5) (width 0.25) (layer "B.Cu") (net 7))
 (segment (start 23.25 9.75) (end 23.25 17.75) (width 0.4) (layer "F.Cu") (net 8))
 (segment (start 23.25 24.25) (end 23.32 24.5) (width 0.4) (layer "F.Cu") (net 8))
 (segment (start 27.6375 5.05) (end 27.5 5) (width 0.4) (layer "F.Cu") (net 8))
 (segment (start 23.25 17.75) (end 23.32 18) (width 0.4) (layer "F.Cu") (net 8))
 (segment (start 22 3.25) (end 21.9375 3.25) (width 0.4) (layer "F.Cu") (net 8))
 (segment (start 22 3) (end 21.975 3.095) (width 0.4) (layer "F.Cu") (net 8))
 (segment (start 21.9375 3) (end 22 3) (width 0.4) (layer "F.Cu") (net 8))
 (segment (start 23.32 18) (end 23.25 18.25) (width 0.4) (layer "F.Cu") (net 8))
 (segment (start 21.975 3.095) (end 22 3.25) (width 0.4) (layer "F.Cu") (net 8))
 (segment (start 27.5 5) (end 26.75 5) (width 0.4) (layer "F.Cu") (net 8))
 (segment (start 23.25 18.25) (end 23.25 24.25) (width 0.4) (layer "F.Cu") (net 8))
 (segment (start 21.9375 3.25) (end 21.9375 3) (width 0.4) (layer "F.Cu") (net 8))
 (segment (start 21.9375 3.25) (end 21.9375 3) (width 0.4) (layer "F.Cu") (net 8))
 (segment (start 28 5) (end 27.6375 5.05) (width 0.4) (layer "F.Cu") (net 8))
 (segment (start 28.5 5) (end 28 5) (width 0.4) (layer "F.Cu") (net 8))
 (via (at 26.75 5) (size 0.7) (drill 0.35) (layers "F.Cu" "B.Cu") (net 8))
 (via (at 22 3) (size 0.7) (drill 0.35) (layers "F.Cu" "B.Cu") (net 8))
 (via (at 28.5 5) (size 0.7) (drill 0.35) (layers "F.Cu" "B.Cu") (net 8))
 (via (at 23.25 9.75) (size 0.7) (drill 0.35) (layers "F.Cu" "B.Cu") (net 8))
 (segment (start 28.5 3.5) (end 28.5 5) (width 0.4) (layer "B.Cu") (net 8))
 (segment (start 26.75 9.75) (end 23.25 9.75) (width 0.4) (layer "B.Cu") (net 8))
 (segment (start 26.75 5) (end 26.75 9.75) (width 0.4) (layer "B.Cu") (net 8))
 (segment (start 12.5 3) (end 22 3) (width 0.4) (layer "B.Cu") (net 8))
 (segment (start 22 3) (end 28.5 3.5) (width 0.4) (layer "B.Cu") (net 8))
 (segment (start 9 33.5) (end 2.5 33.5) (width 0.25) (layer "B.Cu") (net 9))
 (segment (start 9.08 38) (end 9 37.75) (width 0.25) (layer "B.Cu") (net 9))
 (segment (start 2.5 33.5) (end 2.5 24.5) (width 0.25) (layer "B.Cu") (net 9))
 (segment (start 2.5 24.5) (end 3 24.5) (width 0.25) (layer "B.Cu") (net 9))
 (segment (start 9 37.75) (end 9 33.5) (width 0.25) (layer "B.Cu") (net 9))
 (segment (start 4 32) (end 4 30.5) (width 0.25) (layer "F.Cu") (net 10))
 (segment (start 4 32) (end 4 38) (width 0.25) (layer "F.Cu") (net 10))
 (segment (start 13.5 30.5) (end 13.5 31.75) (width 0.25) (layer "F.Cu") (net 10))
 (segment (start 13.5 31.75) (end 13.5875 32) (width 0.25) (layer "F.Cu") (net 10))
 (segment (start 4 30.5) (end 13.5 30.5) (width 0.25) (layer "F.Cu") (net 10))
 (segment (start 20.5 5) (end 25 5) (width 0.25) (layer "F.Cu") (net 11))
 (segment (start 15.4125 32) (end 20.5 32) (width 0.25) (layer "F.Cu") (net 11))
 (segment (start 25 5) (end 25.3625 5.05) (width 0.25) (layer "F.Cu") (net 11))
 (segment (start 20.5 32) (end 20.5 5) (width 0.25) (layer "F.Cu") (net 11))
 (segment (start 9 18) (end 3 18) (width 0.25) (layer "B.Cu") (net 12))
 (segment (start 9.08 32) (end 9 31.75) (width 0.25) (layer "B.Cu") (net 12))
 (segment (start 9 31.75) (end 9 18) (width 0.25) (layer "B.Cu") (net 12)))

